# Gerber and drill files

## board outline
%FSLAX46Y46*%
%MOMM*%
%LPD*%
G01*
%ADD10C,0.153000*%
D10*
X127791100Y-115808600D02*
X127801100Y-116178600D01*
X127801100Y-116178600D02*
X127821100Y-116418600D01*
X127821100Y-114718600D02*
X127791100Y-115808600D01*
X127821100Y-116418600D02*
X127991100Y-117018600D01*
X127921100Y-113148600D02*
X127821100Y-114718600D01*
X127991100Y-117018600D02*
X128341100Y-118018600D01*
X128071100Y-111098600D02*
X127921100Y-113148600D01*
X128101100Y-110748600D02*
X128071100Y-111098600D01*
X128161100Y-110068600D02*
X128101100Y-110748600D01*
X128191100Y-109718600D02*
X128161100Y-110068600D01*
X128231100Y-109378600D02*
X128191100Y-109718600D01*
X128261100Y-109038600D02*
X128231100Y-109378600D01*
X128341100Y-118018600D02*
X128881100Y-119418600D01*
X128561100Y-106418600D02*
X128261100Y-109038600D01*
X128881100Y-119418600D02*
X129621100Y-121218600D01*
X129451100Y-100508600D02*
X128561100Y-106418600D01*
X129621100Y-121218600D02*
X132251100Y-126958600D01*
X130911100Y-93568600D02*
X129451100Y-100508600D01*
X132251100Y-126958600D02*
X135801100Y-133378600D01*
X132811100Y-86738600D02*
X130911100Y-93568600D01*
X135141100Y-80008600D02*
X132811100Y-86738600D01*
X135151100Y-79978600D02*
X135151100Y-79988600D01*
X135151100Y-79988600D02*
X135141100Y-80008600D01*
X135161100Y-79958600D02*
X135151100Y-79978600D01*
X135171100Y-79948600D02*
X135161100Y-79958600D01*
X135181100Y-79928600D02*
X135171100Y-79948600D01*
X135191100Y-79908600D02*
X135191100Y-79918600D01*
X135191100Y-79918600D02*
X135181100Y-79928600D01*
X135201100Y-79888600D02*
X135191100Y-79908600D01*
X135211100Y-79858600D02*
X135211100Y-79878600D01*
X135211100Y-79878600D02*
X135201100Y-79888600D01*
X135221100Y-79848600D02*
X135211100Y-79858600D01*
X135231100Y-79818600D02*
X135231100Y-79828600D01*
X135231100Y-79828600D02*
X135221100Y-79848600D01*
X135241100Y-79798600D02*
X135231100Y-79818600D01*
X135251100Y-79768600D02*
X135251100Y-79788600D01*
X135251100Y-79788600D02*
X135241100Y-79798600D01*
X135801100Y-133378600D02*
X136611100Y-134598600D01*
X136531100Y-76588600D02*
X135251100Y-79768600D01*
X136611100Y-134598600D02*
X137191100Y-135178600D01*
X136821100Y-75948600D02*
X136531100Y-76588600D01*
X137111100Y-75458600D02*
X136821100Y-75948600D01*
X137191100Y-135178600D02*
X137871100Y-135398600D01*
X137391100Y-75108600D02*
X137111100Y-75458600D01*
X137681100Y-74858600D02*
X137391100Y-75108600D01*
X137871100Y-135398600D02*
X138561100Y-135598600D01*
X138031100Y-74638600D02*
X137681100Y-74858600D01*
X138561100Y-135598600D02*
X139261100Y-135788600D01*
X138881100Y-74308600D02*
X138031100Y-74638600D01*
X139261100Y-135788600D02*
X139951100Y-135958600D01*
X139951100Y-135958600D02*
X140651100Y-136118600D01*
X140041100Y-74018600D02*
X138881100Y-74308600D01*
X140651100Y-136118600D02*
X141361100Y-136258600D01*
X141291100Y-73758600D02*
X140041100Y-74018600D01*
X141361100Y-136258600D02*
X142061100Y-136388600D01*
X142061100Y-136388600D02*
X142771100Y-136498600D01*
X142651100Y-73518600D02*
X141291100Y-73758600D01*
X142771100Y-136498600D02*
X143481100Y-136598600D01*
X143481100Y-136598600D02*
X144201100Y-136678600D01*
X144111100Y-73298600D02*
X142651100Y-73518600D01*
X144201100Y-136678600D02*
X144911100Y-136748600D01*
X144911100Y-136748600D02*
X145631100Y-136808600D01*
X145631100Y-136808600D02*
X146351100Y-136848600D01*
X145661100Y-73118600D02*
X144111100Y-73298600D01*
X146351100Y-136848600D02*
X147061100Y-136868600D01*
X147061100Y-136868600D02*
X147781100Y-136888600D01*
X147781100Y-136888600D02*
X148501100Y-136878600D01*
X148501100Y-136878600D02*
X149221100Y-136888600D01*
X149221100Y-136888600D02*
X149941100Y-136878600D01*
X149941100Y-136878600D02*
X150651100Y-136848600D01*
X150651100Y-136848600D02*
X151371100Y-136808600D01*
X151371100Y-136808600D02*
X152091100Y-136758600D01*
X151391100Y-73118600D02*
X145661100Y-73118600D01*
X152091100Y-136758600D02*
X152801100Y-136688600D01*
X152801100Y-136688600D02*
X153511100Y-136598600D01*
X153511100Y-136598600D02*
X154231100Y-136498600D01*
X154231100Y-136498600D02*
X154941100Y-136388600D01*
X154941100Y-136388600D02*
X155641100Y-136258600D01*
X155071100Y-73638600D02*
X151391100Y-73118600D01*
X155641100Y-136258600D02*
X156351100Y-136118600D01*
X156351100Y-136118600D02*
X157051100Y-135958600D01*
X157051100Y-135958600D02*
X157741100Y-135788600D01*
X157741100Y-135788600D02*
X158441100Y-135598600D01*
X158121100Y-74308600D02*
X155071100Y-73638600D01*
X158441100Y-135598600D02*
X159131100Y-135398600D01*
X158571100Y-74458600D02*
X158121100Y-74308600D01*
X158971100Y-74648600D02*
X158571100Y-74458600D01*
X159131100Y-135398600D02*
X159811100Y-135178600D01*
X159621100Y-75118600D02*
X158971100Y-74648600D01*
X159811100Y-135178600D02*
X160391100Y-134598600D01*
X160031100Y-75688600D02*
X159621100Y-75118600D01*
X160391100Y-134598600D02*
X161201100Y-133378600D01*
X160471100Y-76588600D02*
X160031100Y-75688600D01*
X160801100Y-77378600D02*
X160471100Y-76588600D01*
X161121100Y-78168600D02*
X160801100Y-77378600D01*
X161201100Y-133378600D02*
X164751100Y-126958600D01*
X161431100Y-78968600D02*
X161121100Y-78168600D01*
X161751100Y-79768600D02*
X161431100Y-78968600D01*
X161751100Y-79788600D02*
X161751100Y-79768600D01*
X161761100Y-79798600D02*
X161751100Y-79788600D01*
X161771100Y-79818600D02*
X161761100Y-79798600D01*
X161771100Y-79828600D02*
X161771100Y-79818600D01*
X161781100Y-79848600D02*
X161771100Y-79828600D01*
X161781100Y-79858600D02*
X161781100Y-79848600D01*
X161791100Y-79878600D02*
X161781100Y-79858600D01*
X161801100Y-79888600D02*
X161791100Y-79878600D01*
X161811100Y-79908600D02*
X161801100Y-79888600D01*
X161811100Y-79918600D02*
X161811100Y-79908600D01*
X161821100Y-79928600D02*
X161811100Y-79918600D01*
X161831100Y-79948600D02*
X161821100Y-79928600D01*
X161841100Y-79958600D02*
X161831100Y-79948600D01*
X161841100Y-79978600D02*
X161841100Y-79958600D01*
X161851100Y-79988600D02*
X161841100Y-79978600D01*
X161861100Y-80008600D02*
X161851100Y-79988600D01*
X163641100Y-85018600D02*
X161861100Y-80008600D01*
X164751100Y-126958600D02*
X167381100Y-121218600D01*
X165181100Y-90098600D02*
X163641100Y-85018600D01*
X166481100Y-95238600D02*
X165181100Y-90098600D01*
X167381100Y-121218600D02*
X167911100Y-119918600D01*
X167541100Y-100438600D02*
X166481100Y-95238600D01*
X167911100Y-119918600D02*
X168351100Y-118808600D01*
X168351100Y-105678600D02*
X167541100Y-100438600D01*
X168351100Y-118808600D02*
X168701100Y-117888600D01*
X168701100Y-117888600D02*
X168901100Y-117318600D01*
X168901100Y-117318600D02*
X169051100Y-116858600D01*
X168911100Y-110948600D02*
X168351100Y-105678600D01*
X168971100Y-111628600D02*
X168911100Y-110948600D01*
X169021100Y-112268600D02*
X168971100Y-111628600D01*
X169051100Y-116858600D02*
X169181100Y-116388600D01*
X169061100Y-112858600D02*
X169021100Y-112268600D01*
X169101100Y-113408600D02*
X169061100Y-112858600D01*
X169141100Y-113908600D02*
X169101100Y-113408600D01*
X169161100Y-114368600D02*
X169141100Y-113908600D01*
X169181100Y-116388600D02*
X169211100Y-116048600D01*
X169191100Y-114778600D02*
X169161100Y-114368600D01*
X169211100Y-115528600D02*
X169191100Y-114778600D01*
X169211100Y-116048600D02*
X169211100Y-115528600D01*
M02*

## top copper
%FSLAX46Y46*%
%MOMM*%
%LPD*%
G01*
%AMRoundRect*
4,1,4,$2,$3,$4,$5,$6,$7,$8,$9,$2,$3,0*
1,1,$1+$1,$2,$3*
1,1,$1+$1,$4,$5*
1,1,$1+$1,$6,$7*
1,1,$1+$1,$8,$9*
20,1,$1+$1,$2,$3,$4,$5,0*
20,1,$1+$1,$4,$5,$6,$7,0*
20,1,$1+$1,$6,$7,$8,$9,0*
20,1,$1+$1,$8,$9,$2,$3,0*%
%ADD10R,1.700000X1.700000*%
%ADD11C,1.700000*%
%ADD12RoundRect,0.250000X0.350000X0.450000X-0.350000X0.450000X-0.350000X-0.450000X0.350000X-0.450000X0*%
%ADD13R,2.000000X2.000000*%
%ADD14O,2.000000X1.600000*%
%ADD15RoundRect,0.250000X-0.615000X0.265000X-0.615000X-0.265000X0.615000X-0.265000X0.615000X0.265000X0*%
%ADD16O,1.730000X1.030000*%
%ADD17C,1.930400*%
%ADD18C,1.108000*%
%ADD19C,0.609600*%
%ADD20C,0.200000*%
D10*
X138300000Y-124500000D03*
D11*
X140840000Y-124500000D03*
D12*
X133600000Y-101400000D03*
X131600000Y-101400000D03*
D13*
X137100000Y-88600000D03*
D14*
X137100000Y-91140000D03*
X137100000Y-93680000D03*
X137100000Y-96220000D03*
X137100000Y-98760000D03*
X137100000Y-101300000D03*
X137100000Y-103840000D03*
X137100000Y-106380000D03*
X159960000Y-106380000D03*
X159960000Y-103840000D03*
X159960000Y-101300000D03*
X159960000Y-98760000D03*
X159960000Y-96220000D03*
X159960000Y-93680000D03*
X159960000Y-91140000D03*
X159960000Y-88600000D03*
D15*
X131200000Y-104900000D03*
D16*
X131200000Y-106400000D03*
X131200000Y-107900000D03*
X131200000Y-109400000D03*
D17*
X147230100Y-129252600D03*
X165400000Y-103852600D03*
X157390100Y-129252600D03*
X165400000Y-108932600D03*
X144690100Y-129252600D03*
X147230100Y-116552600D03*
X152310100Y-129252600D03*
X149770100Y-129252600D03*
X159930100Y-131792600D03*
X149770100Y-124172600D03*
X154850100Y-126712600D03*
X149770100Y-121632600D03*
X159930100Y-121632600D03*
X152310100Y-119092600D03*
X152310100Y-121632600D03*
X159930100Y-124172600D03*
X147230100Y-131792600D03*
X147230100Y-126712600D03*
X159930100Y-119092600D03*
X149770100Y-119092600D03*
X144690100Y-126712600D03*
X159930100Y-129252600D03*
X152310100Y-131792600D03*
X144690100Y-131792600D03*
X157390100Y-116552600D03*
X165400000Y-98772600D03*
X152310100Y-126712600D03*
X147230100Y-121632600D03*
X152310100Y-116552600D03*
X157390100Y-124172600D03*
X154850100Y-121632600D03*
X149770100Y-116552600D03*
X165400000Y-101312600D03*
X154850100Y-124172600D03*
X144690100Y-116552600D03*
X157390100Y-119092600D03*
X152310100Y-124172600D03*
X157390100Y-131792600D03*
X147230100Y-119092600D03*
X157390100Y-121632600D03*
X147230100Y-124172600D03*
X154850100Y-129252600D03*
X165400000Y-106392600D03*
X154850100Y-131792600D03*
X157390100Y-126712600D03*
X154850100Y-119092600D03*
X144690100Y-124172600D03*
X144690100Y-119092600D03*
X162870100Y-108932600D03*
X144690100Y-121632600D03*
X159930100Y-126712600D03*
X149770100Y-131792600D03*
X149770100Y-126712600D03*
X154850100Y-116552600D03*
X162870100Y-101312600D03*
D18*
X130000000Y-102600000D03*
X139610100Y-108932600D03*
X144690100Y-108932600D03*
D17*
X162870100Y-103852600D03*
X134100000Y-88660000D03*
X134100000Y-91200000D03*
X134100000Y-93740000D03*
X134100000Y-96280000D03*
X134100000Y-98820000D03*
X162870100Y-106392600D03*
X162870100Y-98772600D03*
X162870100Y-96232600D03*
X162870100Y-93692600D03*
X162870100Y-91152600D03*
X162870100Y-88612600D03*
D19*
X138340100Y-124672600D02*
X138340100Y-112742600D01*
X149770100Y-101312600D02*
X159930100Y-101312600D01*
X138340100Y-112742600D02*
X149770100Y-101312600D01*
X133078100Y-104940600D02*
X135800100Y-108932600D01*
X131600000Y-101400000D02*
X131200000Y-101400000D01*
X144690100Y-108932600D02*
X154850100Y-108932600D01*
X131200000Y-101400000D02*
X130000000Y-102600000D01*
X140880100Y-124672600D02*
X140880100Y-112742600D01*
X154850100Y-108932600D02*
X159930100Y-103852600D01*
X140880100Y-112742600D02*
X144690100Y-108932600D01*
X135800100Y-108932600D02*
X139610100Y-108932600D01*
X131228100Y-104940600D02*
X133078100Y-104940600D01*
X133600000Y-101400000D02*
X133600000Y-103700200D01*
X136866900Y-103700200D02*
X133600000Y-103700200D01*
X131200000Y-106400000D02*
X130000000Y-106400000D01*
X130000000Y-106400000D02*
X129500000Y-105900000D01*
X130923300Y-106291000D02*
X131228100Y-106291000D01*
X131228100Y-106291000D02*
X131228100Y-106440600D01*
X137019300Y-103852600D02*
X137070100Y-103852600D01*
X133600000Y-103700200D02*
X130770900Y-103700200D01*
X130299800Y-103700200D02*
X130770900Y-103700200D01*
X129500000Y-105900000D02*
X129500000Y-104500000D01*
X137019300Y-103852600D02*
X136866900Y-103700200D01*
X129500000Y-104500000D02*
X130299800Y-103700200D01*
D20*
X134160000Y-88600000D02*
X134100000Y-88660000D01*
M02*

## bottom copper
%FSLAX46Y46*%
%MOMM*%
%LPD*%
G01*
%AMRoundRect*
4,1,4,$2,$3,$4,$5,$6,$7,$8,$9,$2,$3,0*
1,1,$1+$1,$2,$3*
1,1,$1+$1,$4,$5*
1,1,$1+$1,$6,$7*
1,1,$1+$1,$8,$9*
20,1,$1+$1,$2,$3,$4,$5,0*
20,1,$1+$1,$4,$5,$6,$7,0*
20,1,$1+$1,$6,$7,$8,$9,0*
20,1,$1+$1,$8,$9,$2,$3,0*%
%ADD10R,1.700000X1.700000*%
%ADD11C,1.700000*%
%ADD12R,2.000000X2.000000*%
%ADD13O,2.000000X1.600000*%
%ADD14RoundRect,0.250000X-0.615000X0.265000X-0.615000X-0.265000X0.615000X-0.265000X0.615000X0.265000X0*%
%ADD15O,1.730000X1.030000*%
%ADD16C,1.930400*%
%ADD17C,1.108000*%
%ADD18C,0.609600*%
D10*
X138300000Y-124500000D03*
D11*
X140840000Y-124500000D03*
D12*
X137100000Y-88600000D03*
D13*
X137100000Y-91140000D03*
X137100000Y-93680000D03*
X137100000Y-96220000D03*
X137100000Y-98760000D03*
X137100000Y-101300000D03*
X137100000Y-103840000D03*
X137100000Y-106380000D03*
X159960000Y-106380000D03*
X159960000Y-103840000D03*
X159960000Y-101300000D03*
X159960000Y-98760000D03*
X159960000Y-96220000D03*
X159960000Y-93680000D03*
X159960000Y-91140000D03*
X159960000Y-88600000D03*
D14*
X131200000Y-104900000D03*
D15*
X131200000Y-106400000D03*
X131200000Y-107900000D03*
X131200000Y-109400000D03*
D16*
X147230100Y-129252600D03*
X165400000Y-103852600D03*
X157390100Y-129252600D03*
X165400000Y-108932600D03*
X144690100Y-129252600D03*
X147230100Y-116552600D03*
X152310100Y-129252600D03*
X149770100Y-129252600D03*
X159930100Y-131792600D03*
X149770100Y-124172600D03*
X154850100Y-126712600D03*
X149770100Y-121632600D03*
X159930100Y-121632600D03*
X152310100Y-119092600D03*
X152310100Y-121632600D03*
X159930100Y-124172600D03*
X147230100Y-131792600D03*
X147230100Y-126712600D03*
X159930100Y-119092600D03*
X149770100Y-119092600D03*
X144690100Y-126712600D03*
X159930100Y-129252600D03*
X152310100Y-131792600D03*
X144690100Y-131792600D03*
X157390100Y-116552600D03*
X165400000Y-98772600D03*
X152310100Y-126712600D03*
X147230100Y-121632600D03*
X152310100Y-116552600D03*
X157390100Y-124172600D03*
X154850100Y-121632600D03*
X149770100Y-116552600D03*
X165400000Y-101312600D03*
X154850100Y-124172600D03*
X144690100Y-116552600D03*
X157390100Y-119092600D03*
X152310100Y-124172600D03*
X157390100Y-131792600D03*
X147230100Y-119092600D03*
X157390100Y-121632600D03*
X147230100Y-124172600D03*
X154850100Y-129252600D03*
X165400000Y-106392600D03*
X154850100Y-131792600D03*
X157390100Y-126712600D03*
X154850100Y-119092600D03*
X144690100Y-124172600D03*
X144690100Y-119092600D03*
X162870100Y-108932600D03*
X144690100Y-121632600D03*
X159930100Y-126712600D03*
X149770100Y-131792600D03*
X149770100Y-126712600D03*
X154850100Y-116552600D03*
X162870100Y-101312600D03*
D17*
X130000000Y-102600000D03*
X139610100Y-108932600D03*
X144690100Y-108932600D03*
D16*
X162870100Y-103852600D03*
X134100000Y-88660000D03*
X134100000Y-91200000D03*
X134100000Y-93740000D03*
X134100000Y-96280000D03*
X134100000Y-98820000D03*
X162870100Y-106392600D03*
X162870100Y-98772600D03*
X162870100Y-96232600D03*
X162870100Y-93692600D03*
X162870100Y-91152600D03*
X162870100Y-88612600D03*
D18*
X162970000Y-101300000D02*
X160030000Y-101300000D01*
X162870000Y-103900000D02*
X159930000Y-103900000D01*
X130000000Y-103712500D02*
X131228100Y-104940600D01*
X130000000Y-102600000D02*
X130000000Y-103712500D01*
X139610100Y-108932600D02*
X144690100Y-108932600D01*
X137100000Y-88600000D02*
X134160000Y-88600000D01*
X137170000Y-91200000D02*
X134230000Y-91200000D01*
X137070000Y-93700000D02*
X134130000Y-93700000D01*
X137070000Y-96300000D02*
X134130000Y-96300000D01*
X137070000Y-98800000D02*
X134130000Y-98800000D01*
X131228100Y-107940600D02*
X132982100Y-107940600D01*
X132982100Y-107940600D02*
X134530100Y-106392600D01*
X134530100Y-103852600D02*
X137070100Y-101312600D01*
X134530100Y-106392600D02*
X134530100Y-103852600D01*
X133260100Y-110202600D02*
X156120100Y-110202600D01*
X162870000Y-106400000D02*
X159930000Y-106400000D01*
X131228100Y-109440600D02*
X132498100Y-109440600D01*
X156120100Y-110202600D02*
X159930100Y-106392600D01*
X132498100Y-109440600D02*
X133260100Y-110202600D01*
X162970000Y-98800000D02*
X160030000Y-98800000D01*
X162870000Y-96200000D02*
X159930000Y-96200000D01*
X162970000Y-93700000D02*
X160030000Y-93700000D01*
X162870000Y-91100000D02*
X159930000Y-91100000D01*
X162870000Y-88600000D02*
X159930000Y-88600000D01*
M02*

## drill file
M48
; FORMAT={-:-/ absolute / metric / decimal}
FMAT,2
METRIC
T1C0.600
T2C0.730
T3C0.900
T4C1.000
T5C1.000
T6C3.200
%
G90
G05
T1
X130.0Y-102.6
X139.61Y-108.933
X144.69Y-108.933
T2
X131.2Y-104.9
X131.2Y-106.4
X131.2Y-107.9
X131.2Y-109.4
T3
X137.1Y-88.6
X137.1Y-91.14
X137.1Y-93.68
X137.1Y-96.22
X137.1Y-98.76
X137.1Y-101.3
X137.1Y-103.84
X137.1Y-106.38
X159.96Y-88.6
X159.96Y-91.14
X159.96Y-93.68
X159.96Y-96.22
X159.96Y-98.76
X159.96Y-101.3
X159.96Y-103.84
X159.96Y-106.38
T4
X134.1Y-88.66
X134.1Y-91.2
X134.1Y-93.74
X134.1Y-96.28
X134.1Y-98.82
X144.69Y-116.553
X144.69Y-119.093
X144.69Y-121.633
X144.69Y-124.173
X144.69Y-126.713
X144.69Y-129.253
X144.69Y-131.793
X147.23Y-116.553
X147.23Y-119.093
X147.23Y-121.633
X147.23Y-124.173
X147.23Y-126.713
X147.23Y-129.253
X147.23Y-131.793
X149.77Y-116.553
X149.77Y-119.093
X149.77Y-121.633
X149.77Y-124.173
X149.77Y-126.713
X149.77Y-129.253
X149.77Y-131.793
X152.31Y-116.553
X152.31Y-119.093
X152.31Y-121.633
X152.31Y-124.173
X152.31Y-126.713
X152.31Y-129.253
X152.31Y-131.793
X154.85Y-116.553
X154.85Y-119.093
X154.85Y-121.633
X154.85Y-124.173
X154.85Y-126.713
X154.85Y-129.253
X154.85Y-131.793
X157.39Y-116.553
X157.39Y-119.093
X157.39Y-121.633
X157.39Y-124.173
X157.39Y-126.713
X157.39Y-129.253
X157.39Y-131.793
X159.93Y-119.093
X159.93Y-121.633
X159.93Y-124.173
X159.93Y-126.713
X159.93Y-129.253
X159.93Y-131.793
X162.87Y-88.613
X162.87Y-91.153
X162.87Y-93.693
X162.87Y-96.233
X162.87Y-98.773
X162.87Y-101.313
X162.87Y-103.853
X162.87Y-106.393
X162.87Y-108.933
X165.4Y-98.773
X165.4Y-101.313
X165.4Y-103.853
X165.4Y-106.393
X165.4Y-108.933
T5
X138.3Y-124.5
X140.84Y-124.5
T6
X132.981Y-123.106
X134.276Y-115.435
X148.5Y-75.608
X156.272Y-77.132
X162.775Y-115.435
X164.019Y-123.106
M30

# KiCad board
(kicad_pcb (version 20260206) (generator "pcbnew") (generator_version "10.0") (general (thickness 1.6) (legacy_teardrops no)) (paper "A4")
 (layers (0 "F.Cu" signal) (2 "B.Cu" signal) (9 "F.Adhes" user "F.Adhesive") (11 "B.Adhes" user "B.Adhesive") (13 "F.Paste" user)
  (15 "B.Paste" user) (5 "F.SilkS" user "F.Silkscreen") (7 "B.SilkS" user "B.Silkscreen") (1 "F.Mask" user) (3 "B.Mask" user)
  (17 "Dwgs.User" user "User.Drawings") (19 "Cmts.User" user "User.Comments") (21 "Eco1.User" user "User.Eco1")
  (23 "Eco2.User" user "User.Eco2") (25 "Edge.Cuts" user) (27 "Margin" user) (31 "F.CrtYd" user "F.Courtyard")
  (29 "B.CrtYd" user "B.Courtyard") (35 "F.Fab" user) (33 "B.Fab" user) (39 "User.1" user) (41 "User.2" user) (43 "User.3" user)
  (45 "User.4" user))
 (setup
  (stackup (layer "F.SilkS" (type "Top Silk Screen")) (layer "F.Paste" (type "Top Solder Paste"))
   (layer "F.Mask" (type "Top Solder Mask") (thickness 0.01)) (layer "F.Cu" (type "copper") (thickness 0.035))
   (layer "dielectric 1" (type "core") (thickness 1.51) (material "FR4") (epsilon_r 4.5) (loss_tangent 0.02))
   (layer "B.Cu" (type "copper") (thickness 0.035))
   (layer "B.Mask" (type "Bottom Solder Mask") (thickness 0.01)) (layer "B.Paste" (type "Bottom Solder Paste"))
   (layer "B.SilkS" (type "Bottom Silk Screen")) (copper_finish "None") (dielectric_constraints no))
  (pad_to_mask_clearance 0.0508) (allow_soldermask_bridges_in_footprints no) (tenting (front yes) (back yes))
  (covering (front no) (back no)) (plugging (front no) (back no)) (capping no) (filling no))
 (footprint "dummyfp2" (layer "F.Cu") (at 162.7749 115.435)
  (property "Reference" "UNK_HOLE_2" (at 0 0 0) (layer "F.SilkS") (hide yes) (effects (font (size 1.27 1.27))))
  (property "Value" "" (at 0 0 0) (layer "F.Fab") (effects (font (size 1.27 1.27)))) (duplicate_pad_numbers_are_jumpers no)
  (pad "" np_thru_hole circle (at 0 0) (size 3.2 3.2) (drill 3.2) (layers "*.Cu" "*.Mask")))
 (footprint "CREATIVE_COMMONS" (layer "F.Cu") (at 112.9401 148.3026)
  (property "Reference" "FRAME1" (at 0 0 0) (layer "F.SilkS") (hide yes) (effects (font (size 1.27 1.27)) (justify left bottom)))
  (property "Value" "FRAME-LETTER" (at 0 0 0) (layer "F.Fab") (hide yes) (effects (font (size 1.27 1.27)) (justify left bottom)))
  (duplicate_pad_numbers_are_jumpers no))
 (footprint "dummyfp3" (layer "F.Cu") (at 132.9807 123.1058)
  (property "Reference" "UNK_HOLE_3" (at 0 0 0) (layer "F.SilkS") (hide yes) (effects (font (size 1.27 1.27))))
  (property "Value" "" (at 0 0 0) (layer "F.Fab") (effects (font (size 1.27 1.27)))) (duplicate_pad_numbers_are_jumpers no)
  (pad "" np_thru_hole circle (at 0 0) (size 3.2 3.2) (drill 3.2) (layers "*.Cu" "*.Mask")))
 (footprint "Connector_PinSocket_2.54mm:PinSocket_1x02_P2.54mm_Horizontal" (layer "F.Cu") (at 138.3 124.5 90)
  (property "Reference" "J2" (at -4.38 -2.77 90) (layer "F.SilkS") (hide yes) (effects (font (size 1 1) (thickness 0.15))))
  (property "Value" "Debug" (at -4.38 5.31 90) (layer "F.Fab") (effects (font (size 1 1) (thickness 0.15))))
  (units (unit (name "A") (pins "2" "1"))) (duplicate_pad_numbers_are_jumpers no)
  (pad "1" thru_hole rect (at 0 0 90) (size 1.7 1.7) (drill 1) (layers "*.Cu" "*.Mask") (remove_unused_layers no) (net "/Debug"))
  (pad "2" thru_hole circle (at 0 2.54 90) (size 1.7 1.7) (drill 1) (layers "*.Cu" "*.Mask") (remove_unused_layers no) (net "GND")))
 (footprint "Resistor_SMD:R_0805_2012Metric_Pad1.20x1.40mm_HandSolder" (layer "F.Cu") (at 132.6 101.4 180)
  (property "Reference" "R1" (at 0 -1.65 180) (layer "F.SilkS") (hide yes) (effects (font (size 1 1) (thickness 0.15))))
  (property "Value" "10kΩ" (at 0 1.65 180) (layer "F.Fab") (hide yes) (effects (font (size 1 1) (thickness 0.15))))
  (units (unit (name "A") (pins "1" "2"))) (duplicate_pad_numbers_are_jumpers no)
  (pad "1" smd roundrect (at -1 0 180) (size 1.2 1.4) (layers "F.Cu" "F.Mask" "F.Paste") (roundrect_rratio 0.208333) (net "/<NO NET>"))
  (pad "2" smd roundrect (at 1 0 180) (size 1.2 1.4) (layers "F.Cu" "F.Mask" "F.Paste") (roundrect_rratio 0.208333) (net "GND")))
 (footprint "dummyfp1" (layer "F.Cu") (at 156.2725 77.1318)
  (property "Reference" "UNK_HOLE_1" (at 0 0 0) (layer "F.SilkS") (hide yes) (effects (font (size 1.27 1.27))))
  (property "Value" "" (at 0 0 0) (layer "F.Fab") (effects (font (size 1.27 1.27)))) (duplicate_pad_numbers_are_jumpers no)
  (pad "" np_thru_hole circle (at 0 0) (size 3.2 3.2) (drill 3.2) (layers "*.Cu" "*.Mask")))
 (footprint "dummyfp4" (layer "F.Cu") (at 164.0195 123.1058)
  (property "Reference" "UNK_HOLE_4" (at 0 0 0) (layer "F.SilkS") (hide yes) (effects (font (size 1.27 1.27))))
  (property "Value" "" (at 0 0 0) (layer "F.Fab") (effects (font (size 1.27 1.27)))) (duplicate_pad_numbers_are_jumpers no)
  (pad "" np_thru_hole circle (at 0 0) (size 3.2 3.2) (drill 3.2) (layers "*.Cu" "*.Mask")))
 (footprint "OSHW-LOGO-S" (layer "F.Cu") (at 142.2 77.2)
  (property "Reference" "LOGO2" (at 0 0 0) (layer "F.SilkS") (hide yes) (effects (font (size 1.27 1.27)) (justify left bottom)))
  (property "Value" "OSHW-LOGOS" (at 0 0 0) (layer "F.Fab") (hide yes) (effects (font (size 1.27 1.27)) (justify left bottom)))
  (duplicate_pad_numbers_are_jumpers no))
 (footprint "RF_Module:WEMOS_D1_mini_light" (layer "F.Cu") (at 137.1 88.6)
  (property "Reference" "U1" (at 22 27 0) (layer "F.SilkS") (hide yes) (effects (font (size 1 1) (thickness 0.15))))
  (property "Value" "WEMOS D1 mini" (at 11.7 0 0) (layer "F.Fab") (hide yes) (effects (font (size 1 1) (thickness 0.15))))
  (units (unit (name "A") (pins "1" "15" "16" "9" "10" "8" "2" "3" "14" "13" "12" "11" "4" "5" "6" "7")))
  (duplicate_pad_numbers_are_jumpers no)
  (pad "1" thru_hole rect (at 0 0) (size 2 2) (drill 0.9) (layers "*.Cu" "*.Mask") (remove_unused_layers no)
   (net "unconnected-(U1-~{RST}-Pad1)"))
  (pad "2" thru_hole oval (at 0 2.54) (size 2 1.6) (drill 0.9) (layers "*.Cu" "*.Mask") (remove_unused_layers no)
   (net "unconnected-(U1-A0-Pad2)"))
  (pad "3" thru_hole oval (at 0 5.08) (size 2 1.6) (drill 0.9) (layers "*.Cu" "*.Mask") (remove_unused_layers no)
   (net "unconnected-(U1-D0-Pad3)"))
  (pad "4" thru_hole oval (at 0 7.62) (size 2 1.6) (drill 0.9) (layers "*.Cu" "*.Mask") (remove_unused_layers no)
   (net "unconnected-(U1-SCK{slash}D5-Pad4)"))
  (pad "5" thru_hole oval (at 0 10.16) (size 2 1.6) (drill 0.9) (layers "*.Cu" "*.Mask") (remove_unused_layers no)
   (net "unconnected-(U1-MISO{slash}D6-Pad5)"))
  (pad "6" thru_hole oval (at 0 12.7) (size 2 1.6) (drill 0.9) (layers "*.Cu" "*.Mask") (remove_unused_layers no) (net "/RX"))
  (pad "7" thru_hole oval (at 0 15.24) (size 2 1.6) (drill 0.9) (layers "*.Cu" "*.Mask") (remove_unused_layers no) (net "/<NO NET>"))
  (pad "8" thru_hole oval (at 0 17.78) (size 2 1.6) (drill 0.9) (layers "*.Cu" "*.Mask") (remove_unused_layers no)
   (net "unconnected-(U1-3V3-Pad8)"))
  (pad "9" thru_hole oval (at 22.86 17.78) (size 2 1.6) (drill 0.9) (layers "*.Cu" "*.Mask") (remove_unused_layers no) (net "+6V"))
  (pad "10" thru_hole oval (at 22.86 15.24) (size 2 1.6) (drill 0.9) (layers "*.Cu" "*.Mask") (remove_unused_layers no) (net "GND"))
  (pad "11" thru_hole oval (at 22.86 12.7) (size 2 1.6) (drill 0.9) (layers "*.Cu" "*.Mask") (remove_unused_layers no) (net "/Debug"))
  (pad "12" thru_hole oval (at 22.86 10.16) (size 2 1.6) (drill 0.9) (layers "*.Cu" "*.Mask") (remove_unused_layers no)
   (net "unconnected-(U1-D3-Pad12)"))
  (pad "13" thru_hole oval (at 22.86 7.62) (size 2 1.6) (drill 0.9) (layers "*.Cu" "*.Mask") (remove_unused_layers no)
   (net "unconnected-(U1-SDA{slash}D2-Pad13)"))
  (pad "14" thru_hole oval (at 22.86 5.08) (size 2 1.6) (drill 0.9) (layers "*.Cu" "*.Mask") (remove_unused_layers no)
   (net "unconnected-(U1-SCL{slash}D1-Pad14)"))
  (pad "15" thru_hole oval (at 22.86 2.54) (size 2 1.6) (drill 0.9) (layers "*.Cu" "*.Mask") (remove_unused_layers no)
   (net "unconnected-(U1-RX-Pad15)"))
  (pad "16" thru_hole oval (at 22.86 0) (size 2 1.6) (drill 0.9) (layers "*.Cu" "*.Mask") (remove_unused_layers no)
   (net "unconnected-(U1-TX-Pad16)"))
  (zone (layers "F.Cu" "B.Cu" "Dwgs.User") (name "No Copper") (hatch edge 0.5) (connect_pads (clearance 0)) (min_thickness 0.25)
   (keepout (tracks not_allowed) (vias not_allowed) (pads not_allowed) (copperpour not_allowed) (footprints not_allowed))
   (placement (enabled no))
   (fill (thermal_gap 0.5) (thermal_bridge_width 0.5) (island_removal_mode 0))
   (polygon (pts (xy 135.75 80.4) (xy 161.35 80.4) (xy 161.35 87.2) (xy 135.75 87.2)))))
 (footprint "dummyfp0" (layer "F.Cu") (at 148.5001 75.6078)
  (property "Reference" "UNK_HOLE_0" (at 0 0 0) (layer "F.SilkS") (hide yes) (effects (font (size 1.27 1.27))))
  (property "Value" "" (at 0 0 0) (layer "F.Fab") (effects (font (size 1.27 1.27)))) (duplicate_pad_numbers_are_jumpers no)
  (pad "" np_thru_hole circle (at 0 0) (size 3.2 3.2) (drill 3.2) (layers "*.Cu" "*.Mask")))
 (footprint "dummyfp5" (layer "F.Cu") (at 134.2761 115.435)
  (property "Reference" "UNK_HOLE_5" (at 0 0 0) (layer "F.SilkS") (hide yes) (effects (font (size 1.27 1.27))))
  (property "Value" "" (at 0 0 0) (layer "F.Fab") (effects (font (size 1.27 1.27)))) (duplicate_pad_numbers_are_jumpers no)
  (pad "" np_thru_hole circle (at 0 0) (size 3.2 3.2) (drill 3.2) (layers "*.Cu" "*.Mask")))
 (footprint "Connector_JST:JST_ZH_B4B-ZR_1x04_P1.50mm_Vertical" (layer "B.Cu") (at 131.2 104.9 -90)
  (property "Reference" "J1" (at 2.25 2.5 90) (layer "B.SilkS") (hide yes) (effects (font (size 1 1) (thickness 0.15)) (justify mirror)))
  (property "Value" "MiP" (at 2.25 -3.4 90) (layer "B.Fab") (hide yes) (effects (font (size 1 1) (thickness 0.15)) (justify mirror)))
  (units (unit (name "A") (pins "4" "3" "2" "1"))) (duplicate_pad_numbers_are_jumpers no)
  (pad "1" thru_hole roundrect (at 0 0 270) (size 1.03 1.73) (drill 0.73) (layers "*.Cu" "*.Mask") (remove_unused_layers no)
   (roundrect_rratio 0.242718) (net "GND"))
  (pad "2" thru_hole oval (at 1.5 0 270) (size 1.03 1.73) (drill 0.73) (layers "*.Cu" "*.Mask") (remove_unused_layers no) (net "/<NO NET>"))
  (pad "3" thru_hole oval (at 3 0 270) (size 1.03 1.73) (drill 0.73) (layers "*.Cu" "*.Mask") (remove_unused_layers no) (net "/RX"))
  (pad "4" thru_hole oval (at 4.5 0 270) (size 1.03 1.73) (drill 0.73) (layers "*.Cu" "*.Mask") (remove_unused_layers no) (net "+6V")))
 (gr_line (start 127.7911 115.8086) (end 127.8011 116.1786) (stroke (width 0.153) (type solid)) (layer "Edge.Cuts"))
 (gr_line (start 127.8011 116.1786) (end 127.8211 116.4186) (stroke (width 0.153) (type solid)) (layer "Edge.Cuts"))
 (gr_line (start 127.8211 114.7186) (end 127.7911 115.8086) (stroke (width 0.153) (type solid)) (layer "Edge.Cuts"))
 (gr_line (start 127.8211 116.4186) (end 127.9911 117.0186) (stroke (width 0.153) (type solid)) (layer "Edge.Cuts"))
 (gr_line (start 127.9211 113.1486) (end 127.8211 114.7186) (stroke (width 0.153) (type solid)) (layer "Edge.Cuts"))
 (gr_line (start 127.9911 117.0186) (end 128.3411 118.0186) (stroke (width 0.153) (type solid)) (layer "Edge.Cuts"))
 (gr_line (start 128.0711 111.0986) (end 127.9211 113.1486) (stroke (width 0.153) (type solid)) (layer "Edge.Cuts"))
 (gr_line (start 128.1011 110.7486) (end 128.0711 111.0986) (stroke (width 0.153) (type solid)) (layer "Edge.Cuts"))
 (gr_line (start 128.1611 110.0686) (end 128.1011 110.7486) (stroke (width 0.153) (type solid)) (layer "Edge.Cuts"))
 (gr_line (start 128.1911 109.7186) (end 128.1611 110.0686) (stroke (width 0.153) (type solid)) (layer "Edge.Cuts"))
 (gr_line (start 128.2311 109.3786) (end 128.1911 109.7186) (stroke (width 0.153) (type solid)) (layer "Edge.Cuts"))
 (gr_line (start 128.2611 109.0386) (end 128.2311 109.3786) (stroke (width 0.153) (type solid)) (layer "Edge.Cuts"))
 (gr_line (start 128.3411 118.0186) (end 128.8811 119.4186) (stroke (width 0.153) (type solid)) (layer "Edge.Cuts"))
 (gr_line (start 128.5611 106.4186) (end 128.2611 109.0386) (stroke (width 0.153) (type solid)) (layer "Edge.Cuts"))
 (gr_line (start 128.8811 119.4186) (end 129.6211 121.2186) (stroke (width 0.153) (type solid)) (layer "Edge.Cuts"))
 (gr_line (start 129.4511 100.5086) (end 128.5611 106.4186) (stroke (width 0.153) (type solid)) (layer "Edge.Cuts"))
 (gr_line (start 129.6211 121.2186) (end 132.2511 126.9586) (stroke (width 0.153) (type solid)) (layer "Edge.Cuts"))
 (gr_line (start 130.9111 93.5686) (end 129.4511 100.5086) (stroke (width 0.153) (type solid)) (layer "Edge.Cuts"))
 (gr_line (start 132.2511 126.9586) (end 135.8011 133.3786) (stroke (width 0.153) (type solid)) (layer "Edge.Cuts"))
 (gr_line (start 132.8111 86.7386) (end 130.9111 93.5686) (stroke (width 0.153) (type solid)) (layer "Edge.Cuts"))
 (gr_line (start 135.1411 80.0086) (end 132.8111 86.7386) (stroke (width 0.153) (type solid)) (layer "Edge.Cuts"))
 (gr_line (start 135.1511 79.9786) (end 135.1511 79.9886) (stroke (width 0.153) (type solid)) (layer "Edge.Cuts"))
 (gr_line (start 135.1511 79.9886) (end 135.1411 80.0086) (stroke (width 0.153) (type solid)) (layer "Edge.Cuts"))
 (gr_line (start 135.1611 79.9586) (end 135.1511 79.9786) (stroke (width 0.153) (type solid)) (layer "Edge.Cuts"))
 (gr_line (start 135.1711 79.9486) (end 135.1611 79.9586) (stroke (width 0.153) (type solid)) (layer "Edge.Cuts"))
 (gr_line (start 135.1811 79.9286) (end 135.1711 79.9486) (stroke (width 0.153) (type solid)) (layer "Edge.Cuts"))
 (gr_line (start 135.1911 79.9086) (end 135.1911 79.9186) (stroke (width 0.153) (type solid)) (layer "Edge.Cuts"))
 (gr_line (start 135.1911 79.9186) (end 135.1811 79.9286) (stroke (width 0.153) (type solid)) (layer "Edge.Cuts"))
 (gr_line (start 135.2011 79.8886) (end 135.1911 79.9086) (stroke (width 0.153) (type solid)) (layer "Edge.Cuts"))
 (gr_line (start 135.2111 79.8586) (end 135.2111 79.8786) (stroke (width 0.153) (type solid)) (layer "Edge.Cuts"))
 (gr_line (start 135.2111 79.8786) (end 135.2011 79.8886) (stroke (width 0.153) (type solid)) (layer "Edge.Cuts"))
 (gr_line (start 135.2211 79.8486) (end 135.2111 79.8586) (stroke (width 0.153) (type solid)) (layer "Edge.Cuts"))
 (gr_line (start 135.2311 79.8186) (end 135.2311 79.8286) (stroke (width 0.153) (type solid)) (layer "Edge.Cuts"))
 (gr_line (start 135.2311 79.8286) (end 135.2211 79.8486) (stroke (width 0.153) (type solid)) (layer "Edge.Cuts"))
 (gr_line (start 135.2411 79.7986) (end 135.2311 79.8186) (stroke (width 0.153) (type solid)) (layer "Edge.Cuts"))
 (gr_line (start 135.2511 79.7686) (end 135.2511 79.7886) (stroke (width 0.153) (type solid)) (layer "Edge.Cuts"))
 (gr_line (start 135.2511 79.7886) (end 135.2411 79.7986) (stroke (width 0.153) (type solid)) (layer "Edge.Cuts"))
 (gr_line (start 135.8011 133.3786) (end 136.6111 134.5986) (stroke (width 0.153) (type solid)) (layer "Edge.Cuts"))
 (gr_line (start 136.5311 76.5886) (end 135.2511 79.7686) (stroke (width 0.153) (type solid)) (layer "Edge.Cuts"))
 (gr_line (start 136.6111 134.5986) (end 137.1911 135.1786) (stroke (width 0.153) (type solid)) (layer "Edge.Cuts"))
 (gr_line (start 136.8211 75.9486) (end 136.5311 76.5886) (stroke (width 0.153) (type solid)) (layer "Edge.Cuts"))
 (gr_line (start 137.1111 75.4586) (end 136.8211 75.9486) (stroke (width 0.153) (type solid)) (layer "Edge.Cuts"))
 (gr_line (start 137.1911 135.1786) (end 137.8711 135.3986) (stroke (width 0.153) (type solid)) (layer "Edge.Cuts"))
 (gr_line (start 137.3911 75.1086) (end 137.1111 75.4586) (stroke (width 0.153) (type solid)) (layer "Edge.Cuts"))
 (gr_line (start 137.6811 74.8586) (end 137.3911 75.1086) (stroke (width 0.153) (type solid)) (layer "Edge.Cuts"))
 (gr_line (start 137.8711 135.3986) (end 138.5611 135.5986) (stroke (width 0.153) (type solid)) (layer "Edge.Cuts"))
 (gr_line (start 138.0311 74.6386) (end 137.6811 74.8586) (stroke (width 0.153) (type solid)) (layer "Edge.Cuts"))
 (gr_line (start 138.5611 135.5986) (end 139.2611 135.7886) (stroke (width 0.153) (type solid)) (layer "Edge.Cuts"))
 (gr_line (start 138.8811 74.3086) (end 138.0311 74.6386) (stroke (width 0.153) (type solid)) (layer "Edge.Cuts"))
 (gr_line (start 139.2611 135.7886) (end 139.9511 135.9586) (stroke (width 0.153) (type solid)) (layer "Edge.Cuts"))
 (gr_line (start 139.9511 135.9586) (end 140.6511 136.1186) (stroke (width 0.153) (type solid)) (layer "Edge.Cuts"))
 (gr_line (start 140.0411 74.0186) (end 138.8811 74.3086) (stroke (width 0.153) (type solid)) (layer "Edge.Cuts"))
 (gr_line (start 140.6511 136.1186) (end 141.3611 136.2586) (stroke (width 0.153) (type solid)) (layer "Edge.Cuts"))
 (gr_line (start 141.2911 73.7586) (end 140.0411 74.0186) (stroke (width 0.153) (type solid)) (layer "Edge.Cuts"))
 (gr_line (start 141.3611 136.2586) (end 142.0611 136.3886) (stroke (width 0.153) (type solid)) (layer "Edge.Cuts"))
 (gr_line (start 142.0611 136.3886) (end 142.7711 136.4986) (stroke (width 0.153) (type solid)) (layer "Edge.Cuts"))
 (gr_line (start 142.6511 73.5186) (end 141.2911 73.7586) (stroke (width 0.153) (type solid)) (layer "Edge.Cuts"))
 (gr_line (start 142.7711 136.4986) (end 143.4811 136.5986) (stroke (width 0.153) (type solid)) (layer "Edge.Cuts"))
 (gr_line (start 143.4811 136.5986) (end 144.2011 136.6786) (stroke (width 0.153) (type solid)) (layer "Edge.Cuts"))
 (gr_line (start 144.1111 73.2986) (end 142.6511 73.5186) (stroke (width 0.153) (type solid)) (layer "Edge.Cuts"))
 (gr_line (start 144.2011 136.6786) (end 144.9111 136.7486) (stroke (width 0.153) (type solid)) (layer "Edge.Cuts"))
 (gr_line (start 144.9111 136.7486) (end 145.6311 136.8086) (stroke (width 0.153) (type solid)) (layer "Edge.Cuts"))
 (gr_line (start 145.6311 136.8086) (end 146.3511 136.8486) (stroke (width 0.153) (type solid)) (layer "Edge.Cuts"))
 (gr_line (start 145.6611 73.1186) (end 144.1111 73.2986) (stroke (width 0.153) (type solid)) (layer "Edge.Cuts"))
 (gr_line (start 146.3511 136.8486) (end 147.0611 136.8686) (stroke (width 0.153) (type solid)) (layer "Edge.Cuts"))
 (gr_line (start 147.0611 136.8686) (end 147.7811 136.8886) (stroke (width 0.153) (type solid)) (layer "Edge.Cuts"))
 (gr_line (start 147.7811 136.8886) (end 148.5011 136.8786) (stroke (width 0.153) (type solid)) (layer "Edge.Cuts"))
 (gr_line (start 148.5011 136.8786) (end 149.2211 136.8886) (stroke (width 0.153) (type solid)) (layer "Edge.Cuts"))
 (gr_line (start 149.2211 136.8886) (end 149.9411 136.8786) (stroke (width 0.153) (type solid)) (layer "Edge.Cuts"))
 (gr_line (start 149.9411 136.8786) (end 150.6511 136.8486) (stroke (width 0.153) (type solid)) (layer "Edge.Cuts"))
 (gr_line (start 150.6511 136.8486) (end 151.3711 136.8086) (stroke (width 0.153) (type solid)) (layer "Edge.Cuts"))
 (gr_line (start 151.3711 136.8086) (end 152.0911 136.7586) (stroke (width 0.153) (type solid)) (layer "Edge.Cuts"))
 (gr_line (start 151.3911 73.1186) (end 145.6611 73.1186) (stroke (width 0.153) (type solid)) (layer "Edge.Cuts"))
 (gr_line (start 152.0911 136.7586) (end 152.8011 136.6886) (stroke (width 0.153) (type solid)) (layer "Edge.Cuts"))
 (gr_line (start 152.8011 136.6886) (end 153.5111 136.5986) (stroke (width 0.153) (type solid)) (layer "Edge.Cuts"))
 (gr_line (start 153.5111 136.5986) (end 154.2311 136.4986) (stroke (width 0.153) (type solid)) (layer "Edge.Cuts"))
 (gr_line (start 154.2311 136.4986) (end 154.9411 136.3886) (stroke (width 0.153) (type solid)) (layer "Edge.Cuts"))
 (gr_line (start 154.9411 136.3886) (end 155.6411 136.2586) (stroke (width 0.153) (type solid)) (layer "Edge.Cuts"))
 (gr_line (start 155.0711 73.6386) (end 151.3911 73.1186) (stroke (width 0.153) (type solid)) (layer "Edge.Cuts"))
 (gr_line (start 155.6411 136.2586) (end 156.3511 136.1186) (stroke (width 0.153) (type solid)) (layer "Edge.Cuts"))
 (gr_line (start 156.3511 136.1186) (end 157.0511 135.9586) (stroke (width 0.153) (type solid)) (layer "Edge.Cuts"))
 (gr_line (start 157.0511 135.9586) (end 157.7411 135.7886) (stroke (width 0.153) (type solid)) (layer "Edge.Cuts"))
 (gr_line (start 157.7411 135.7886) (end 158.4411 135.5986) (stroke (width 0.153) (type solid)) (layer "Edge.Cuts"))
 (gr_line (start 158.1211 74.3086) (end 155.0711 73.6386) (stroke (width 0.153) (type solid)) (layer "Edge.Cuts"))
 (gr_line (start 158.4411 135.5986) (end 159.1311 135.3986) (stroke (width 0.153) (type solid)) (layer "Edge.Cuts"))
 (gr_line (start 158.5711 74.4586) (end 158.1211 74.3086) (stroke (width 0.153) (type solid)) (layer "Edge.Cuts"))
 (gr_line (start 158.9711 74.6486) (end 158.5711 74.4586) (stroke (width 0.153) (type solid)) (layer "Edge.Cuts"))
 (gr_line (start 159.1311 135.3986) (end 159.8111 135.1786) (stroke (width 0.153) (type solid)) (layer "Edge.Cuts"))
 (gr_line (start 159.6211 75.1186) (end 158.9711 74.6486) (stroke (width 0.153) (type solid)) (layer "Edge.Cuts"))
 (gr_line (start 159.8111 135.1786) (end 160.3911 134.5986) (stroke (width 0.153) (type solid)) (layer "Edge.Cuts"))
 (gr_line (start 160.0311 75.6886) (end 159.6211 75.1186) (stroke (width 0.153) (type solid)) (layer "Edge.Cuts"))
 (gr_line (start 160.3911 134.5986) (end 161.2011 133.3786) (stroke (width 0.153) (type solid)) (layer "Edge.Cuts"))
 (gr_line (start 160.4711 76.5886) (end 160.0311 75.6886) (stroke (width 0.153) (type solid)) (layer "Edge.Cuts"))
 (gr_line (start 160.8011 77.3786) (end 160.4711 76.5886) (stroke (width 0.153) (type solid)) (layer "Edge.Cuts"))
 (gr_line (start 161.1211 78.1686) (end 160.8011 77.3786) (stroke (width 0.153) (type solid)) (layer "Edge.Cuts"))
 (gr_line (start 161.2011 133.3786) (end 164.7511 126.9586) (stroke (width 0.153) (type solid)) (layer "Edge.Cuts"))
 (gr_line (start 161.4311 78.9686) (end 161.1211 78.1686) (stroke (width 0.153) (type solid)) (layer "Edge.Cuts"))
 (gr_line (start 161.7511 79.7686) (end 161.4311 78.9686) (stroke (width 0.153) (type solid)) (layer "Edge.Cuts"))
 (gr_line (start 161.7511 79.7886) (end 161.7511 79.7686) (stroke (width 0.153) (type solid)) (layer "Edge.Cuts"))
 (gr_line (start 161.7611 79.7986) (end 161.7511 79.7886) (stroke (width 0.153) (type solid)) (layer "Edge.Cuts"))
 (gr_line (start 161.7711 79.8186) (end 161.7611 79.7986) (stroke (width 0.153) (type solid)) (layer "Edge.Cuts"))
 (gr_line (start 161.7711 79.8286) (end 161.7711 79.8186) (stroke (width 0.153) (type solid)) (layer "Edge.Cuts"))
 (gr_line (start 161.7811 79.8486) (end 161.7711 79.8286) (stroke (width 0.153) (type solid)) (layer "Edge.Cuts"))
 (gr_line (start 161.7811 79.8586) (end 161.7811 79.8486) (stroke (width 0.153) (type solid)) (layer "Edge.Cuts"))
 (gr_line (start 161.7911 79.8786) (end 161.7811 79.8586) (stroke (width 0.153) (type solid)) (layer "Edge.Cuts"))
 (gr_line (start 161.8011 79.8886) (end 161.7911 79.8786) (stroke (width 0.153) (type solid)) (layer "Edge.Cuts"))
 (gr_line (start 161.8111 79.9086) (end 161.8011 79.8886) (stroke (width 0.153) (type solid)) (layer "Edge.Cuts"))
 (gr_line (start 161.8111 79.9186) (end 161.8111 79.9086) (stroke (width 0.153) (type solid)) (layer "Edge.Cuts"))
 (gr_line (start 161.8211 79.9286) (end 161.8111 79.9186) (stroke (width 0.153) (type solid)) (layer "Edge.Cuts"))
 (gr_line (start 161.8311 79.9486) (end 161.8211 79.9286) (stroke (width 0.153) (type solid)) (layer "Edge.Cuts"))
 (gr_line (start 161.8411 79.9586) (end 161.8311 79.9486) (stroke (width 0.153) (type solid)) (layer "Edge.Cuts"))
 (gr_line (start 161.8411 79.9786) (end 161.8411 79.9586) (stroke (width 0.153) (type solid)) (layer "Edge.Cuts"))
 (gr_line (start 161.8511 79.9886) (end 161.8411 79.9786) (stroke (width 0.153) (type solid)) (layer "Edge.Cuts"))
 (gr_line (start 161.8611 80.0086) (end 161.8511 79.9886) (stroke (width 0.153) (type solid)) (layer "Edge.Cuts"))
 (gr_line (start 163.6411 85.0186) (end 161.8611 80.0086) (stroke (width 0.153) (type solid)) (layer "Edge.Cuts"))
 (gr_line (start 164.7511 126.9586) (end 167.3811 121.2186) (stroke (width 0.153) (type solid)) (layer "Edge.Cuts"))
 (gr_line (start 165.1811 90.0986) (end 163.6411 85.0186) (stroke (width 0.153) (type solid)) (layer "Edge.Cuts"))
 (gr_line (start 166.4811 95.2386) (end 165.1811 90.0986) (stroke (width 0.153) (type solid)) (layer "Edge.Cuts"))
 (gr_line (start 167.3811 121.2186) (end 167.9111 119.9186) (stroke (width 0.153) (type solid)) (layer "Edge.Cuts"))
 (gr_line (start 167.5411 100.4386) (end 166.4811 95.2386) (stroke (width 0.153) (type solid)) (layer "Edge.Cuts"))
 (gr_line (start 167.9111 119.9186) (end 168.3511 118.8086) (stroke (width 0.153) (type solid)) (layer "Edge.Cuts"))
 (gr_line (start 168.3511 105.6786) (end 167.5411 100.4386) (stroke (width 0.153) (type solid)) (layer "Edge.Cuts"))
 (gr_line (start 168.3511 118.8086) (end 168.7011 117.8886) (stroke (width 0.153) (type solid)) (layer "Edge.Cuts"))
 (gr_line (start 168.7011 117.8886) (end 168.9011 117.3186) (stroke (width 0.153) (type solid)) (layer "Edge.Cuts"))
 (gr_line (start 168.9011 117.3186) (end 169.0511 116.8586) (stroke (width 0.153) (type solid)) (layer "Edge.Cuts"))
 (gr_line (start 168.9111 110.9486) (end 168.3511 105.6786) (stroke (width 0.153) (type solid)) (layer "Edge.Cuts"))
 (gr_line (start 168.9711 111.6286) (end 168.9111 110.9486) (stroke (width 0.153) (type solid)) (layer "Edge.Cuts"))
 (gr_line (start 169.0211 112.2686) (end 168.9711 111.6286) (stroke (width 0.153) (type solid)) (layer "Edge.Cuts"))
 (gr_line (start 169.0511 116.8586) (end 169.1811 116.3886) (stroke (width 0.153) (type solid)) (layer "Edge.Cuts"))
 (gr_line (start 169.0611 112.8586) (end 169.0211 112.2686) (stroke (width 0.153) (type solid)) (layer "Edge.Cuts"))
 (gr_line (start 169.1011 113.4086) (end 169.0611 112.8586) (stroke (width 0.153) (type solid)) (layer "Edge.Cuts"))
 (gr_line (start 169.1411 113.9086) (end 169.1011 113.4086) (stroke (width 0.153) (type solid)) (layer "Edge.Cuts"))
 (gr_line (start 169.1611 114.3686) (end 169.1411 113.9086) (stroke (width 0.153) (type solid)) (layer "Edge.Cuts"))
 (gr_line (start 169.1811 116.3886) (end 169.2111 116.0486) (stroke (width 0.153) (type solid)) (layer "Edge.Cuts"))
 (gr_line (start 169.1911 114.7786) (end 169.1611 114.3686) (stroke (width 0.153) (type solid)) (layer "Edge.Cuts"))
 (gr_line (start 169.2111 115.5286) (end 169.1911 114.7786) (stroke (width 0.153) (type solid)) (layer "Edge.Cuts"))
 (gr_line (start 169.2111 116.0486) (end 169.2111 115.5286) (stroke (width 0.153) (type solid)) (layer "Edge.Cuts"))
 (via (at 147.2301 129.2526) (size 1.9304) (drill 1) (layers "F.Cu" "B.Cu") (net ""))
 (via (at 165.4 103.8526) (size 1.9304) (drill 1) (layers "F.Cu" "B.Cu") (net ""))
 (via (at 157.3901 129.2526) (size 1.9304) (drill 1) (layers "F.Cu" "B.Cu") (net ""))
 (via (at 165.4 108.9326) (size 1.9304) (drill 1) (layers "F.Cu" "B.Cu") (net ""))
 (via (at 144.6901 129.2526) (size 1.9304) (drill 1) (layers "F.Cu" "B.Cu") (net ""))
 (via (at 147.2301 116.5526) (size 1.9304) (drill 1) (layers "F.Cu" "B.Cu") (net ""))
 (via (at 152.3101 129.2526) (size 1.9304) (drill 1) (layers "F.Cu" "B.Cu") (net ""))
 (via (at 149.7701 129.2526) (size 1.9304) (drill 1) (layers "F.Cu" "B.Cu") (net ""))
 (via (at 159.9301 131.7926) (size 1.9304) (drill 1) (layers "F.Cu" "B.Cu") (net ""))
 (via (at 149.7701 124.1726) (size 1.9304) (drill 1) (layers "F.Cu" "B.Cu") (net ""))
 (via (at 154.8501 126.7126) (size 1.9304) (drill 1) (layers "F.Cu" "B.Cu") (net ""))
 (via (at 149.7701 121.6326) (size 1.9304) (drill 1) (layers "F.Cu" "B.Cu") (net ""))
 (via (at 159.9301 121.6326) (size 1.9304) (drill 1) (layers "F.Cu" "B.Cu") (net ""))
 (via (at 152.3101 119.0926) (size 1.9304) (drill 1) (layers "F.Cu" "B.Cu") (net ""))
 (via (at 152.3101 121.6326) (size 1.9304) (drill 1) (layers "F.Cu" "B.Cu") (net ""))
 (via (at 159.9301 124.1726) (size 1.9304) (drill 1) (layers "F.Cu" "B.Cu") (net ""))
 (via (at 147.2301 131.7926) (size 1.9304) (drill 1) (layers "F.Cu" "B.Cu") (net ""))
 (via (at 147.2301 126.7126) (size 1.9304) (drill 1) (layers "F.Cu" "B.Cu") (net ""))
 (via (at 159.9301 119.0926) (size 1.9304) (drill 1) (layers "F.Cu" "B.Cu") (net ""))
 (via (at 149.7701 119.0926) (size 1.9304) (drill 1) (layers "F.Cu" "B.Cu") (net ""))
 (via (at 144.6901 126.7126) (size 1.9304) (drill 1) (layers "F.Cu" "B.Cu") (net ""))
 (via (at 159.9301 129.2526) (size 1.9304) (drill 1) (layers "F.Cu" "B.Cu") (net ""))
 (via (at 152.3101 131.7926) (size 1.9304) (drill 1) (layers "F.Cu" "B.Cu") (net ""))
 (via (at 144.6901 131.7926) (size 1.9304) (drill 1) (layers "F.Cu" "B.Cu") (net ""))
 (via (at 157.3901 116.5526) (size 1.9304) (drill 1) (layers "F.Cu" "B.Cu") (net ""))
 (via (at 165.4 98.7726) (size 1.9304) (drill 1) (layers "F.Cu" "B.Cu") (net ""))
 (via (at 152.3101 126.7126) (size 1.9304) (drill 1) (layers "F.Cu" "B.Cu") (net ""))
 (via (at 147.2301 121.6326) (size 1.9304) (drill 1) (layers "F.Cu" "B.Cu") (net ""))
 (via (at 152.3101 116.5526) (size 1.9304) (drill 1) (layers "F.Cu" "B.Cu") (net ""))
 (via (at 157.3901 124.1726) (size 1.9304) (drill 1) (layers "F.Cu" "B.Cu") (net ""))
 (via (at 154.8501 121.6326) (size 1.9304) (drill 1) (layers "F.Cu" "B.Cu") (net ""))
 (via (at 149.7701 116.5526) (size 1.9304) (drill 1) (layers "F.Cu" "B.Cu") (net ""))
 (via (at 165.4 101.3126) (size 1.9304) (drill 1) (layers "F.Cu" "B.Cu") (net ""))
 (via (at 154.8501 124.1726) (size 1.9304) (drill 1) (layers "F.Cu" "B.Cu") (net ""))
 (via (at 144.6901 116.5526) (size 1.9304) (drill 1) (layers "F.Cu" "B.Cu") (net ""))
 (via (at 157.3901 119.0926) (size 1.9304) (drill 1) (layers "F.Cu" "B.Cu") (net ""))
 (via (at 152.3101 124.1726) (size 1.9304) (drill 1) (layers "F.Cu" "B.Cu") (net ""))
 (via (at 157.3901 131.7926) (size 1.9304) (drill 1) (layers "F.Cu" "B.Cu") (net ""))
 (via (at 147.2301 119.0926) (size 1.9304) (drill 1) (layers "F.Cu" "B.Cu") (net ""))
 (via (at 157.3901 121.6326) (size 1.9304) (drill 1) (layers "F.Cu" "B.Cu") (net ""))
 (via (at 147.2301 124.1726) (size 1.9304) (drill 1) (layers "F.Cu" "B.Cu") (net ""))
 (via (at 154.8501 129.2526) (size 1.9304) (drill 1) (layers "F.Cu" "B.Cu") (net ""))
 (via (at 165.4 106.3926) (size 1.9304) (drill 1) (layers "F.Cu" "B.Cu") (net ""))
 (via (at 154.8501 131.7926) (size 1.9304) (drill 1) (layers "F.Cu" "B.Cu") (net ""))
 (via (at 157.3901 126.7126) (size 1.9304) (drill 1) (layers "F.Cu" "B.Cu") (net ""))
 (via (at 154.8501 119.0926) (size 1.9304) (drill 1) (layers "F.Cu" "B.Cu") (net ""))
 (via (at 144.6901 124.1726) (size 1.9304) (drill 1) (layers "F.Cu" "B.Cu") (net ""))
 (via (at 144.6901 119.0926) (size 1.9304) (drill 1) (layers "F.Cu" "B.Cu") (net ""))
 (via (at 162.8701 108.9326) (size 1.9304) (drill 1) (layers "F.Cu" "B.Cu") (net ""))
 (via (at 144.6901 121.6326) (size 1.9304) (drill 1) (layers "F.Cu" "B.Cu") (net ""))
 (via (at 159.9301 126.7126) (size 1.9304) (drill 1) (layers "F.Cu" "B.Cu") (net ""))
 (via (at 149.7701 131.7926) (size 1.9304) (drill 1) (layers "F.Cu" "B.Cu") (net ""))
 (via (at 149.7701 126.7126) (size 1.9304) (drill 1) (layers "F.Cu" "B.Cu") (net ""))
 (via (at 154.8501 116.5526) (size 1.9304) (drill 1) (layers "F.Cu" "B.Cu") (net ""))
 (segment (start 138.3401 124.6726) (end 138.3401 112.7426) (width 0.6096) (layer "F.Cu") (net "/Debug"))
 (segment (start 149.7701 101.3126) (end 159.9301 101.3126) (width 0.6096) (layer "F.Cu") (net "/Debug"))
 (segment (start 138.3401 112.7426) (end 149.7701 101.3126) (width 0.6096) (layer "F.Cu") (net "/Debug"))
 (via (at 162.8701 101.3126) (size 1.9304) (drill 1) (layers "F.Cu" "B.Cu") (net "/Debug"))
 (segment (start 162.97 101.3) (end 160.03 101.3) (width 0.6096) (layer "B.Cu") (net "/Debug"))
 (segment (start 133.0781 104.9406) (end 135.8001 108.9326) (width 0.6096) (layer "F.Cu") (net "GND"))
 (segment (start 131.6 101.4) (end 131.2 101.4) (width 0.6096) (layer "F.Cu") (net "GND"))
 (segment (start 144.6901 108.9326) (end 154.8501 108.9326) (width 0.6096) (layer "F.Cu") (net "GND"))
 (segment (start 131.2 101.4) (end 130 102.6) (width 0.6096) (layer "F.Cu") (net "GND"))
 (segment (start 140.8801 124.6726) (end 140.8801 112.7426) (width 0.6096) (layer "F.Cu") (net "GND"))
 (segment (start 154.8501 108.9326) (end 159.9301 103.8526) (width 0.6096) (layer "F.Cu") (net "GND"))
 (segment (start 140.8801 112.7426) (end 144.6901 108.9326) (width 0.6096) (layer "F.Cu") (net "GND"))
 (segment (start 135.8001 108.9326) (end 139.6101 108.9326) (width 0.6096) (layer "F.Cu") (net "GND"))
 (segment (start 131.2281 104.9406) (end 133.0781 104.9406) (width 0.6096) (layer "F.Cu") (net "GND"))
 (via (at 130 102.6) (size 1.108) (drill 0.6) (layers "F.Cu" "B.Cu") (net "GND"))
 (via (at 139.6101 108.9326) (size 1.108) (drill 0.6) (layers "F.Cu" "B.Cu") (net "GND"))
 (via (at 144.6901 108.9326) (size 1.108) (drill 0.6) (layers "F.Cu" "B.Cu") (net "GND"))
 (via (at 162.8701 103.8526) (size 1.9304) (drill 1) (layers "F.Cu" "B.Cu") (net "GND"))
 (segment (start 162.87 103.9) (end 159.93 103.9) (width 0.6096) (layer "B.Cu") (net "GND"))
 (segment (start 130 103.7125) (end 131.2281 104.9406) (width 0.6096) (layer "B.Cu") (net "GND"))
 (segment (start 130 102.6) (end 130 103.7125) (width 0.6096) (layer "B.Cu") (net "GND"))
 (segment (start 139.6101 108.9326) (end 144.6901 108.9326) (width 0.6096) (layer "B.Cu") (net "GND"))
 (segment (start 133.6 101.4) (end 133.6 103.7002) (width 0.6096) (layer "F.Cu") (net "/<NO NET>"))
 (segment (start 136.8669 103.7002) (end 133.6 103.7002) (width 0.6096) (layer "F.Cu") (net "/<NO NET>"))
 (segment (start 131.2 106.4) (end 130 106.4) (width 0.6096) (layer "F.Cu") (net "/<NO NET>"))
 (segment (start 130 106.4) (end 129.5 105.9) (width 0.6096) (layer "F.Cu") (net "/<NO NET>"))
 (segment (start 130.9233 106.291) (end 131.2281 106.291) (width 0.6096) (layer "F.Cu") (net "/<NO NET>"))
 (segment (start 131.2281 106.291) (end 131.2281 106.4406) (width 0.6096) (layer "F.Cu") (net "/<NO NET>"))
 (segment (start 137.0193 103.8526) (end 137.0701 103.8526) (width 0.6096) (layer "F.Cu") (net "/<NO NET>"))
 (segment (start 133.6 103.7002) (end 130.7709 103.7002) (width 0.6096) (layer "F.Cu") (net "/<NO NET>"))
 (segment (start 130.2998 103.7002) (end 130.7709 103.7002) (width 0.6096) (layer "F.Cu") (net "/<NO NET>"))
 (segment (start 129.5 105.9) (end 129.5 104.5) (width 0.6096) (layer "F.Cu") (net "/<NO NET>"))
 (segment (start 137.0193 103.8526) (end 136.8669 103.7002) (width 0.6096) (layer "F.Cu") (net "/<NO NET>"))
 (segment (start 129.5 104.5) (end 130.2998 103.7002) (width 0.6096) (layer "F.Cu") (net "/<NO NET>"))
 (segment (start 134.16 88.6) (end 134.1 88.66) (width 0.2) (layer "F.Cu") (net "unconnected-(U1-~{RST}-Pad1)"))
 (via (at 134.1 88.66) (size 1.9304) (drill 1) (layers "F.Cu" "B.Cu") (free yes) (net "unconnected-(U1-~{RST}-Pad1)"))
 (segment (start 137.1 88.6) (end 134.16 88.6) (width 0.6096) (layer "B.Cu") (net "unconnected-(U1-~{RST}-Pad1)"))
 (via (at 134.1 91.2) (size 1.9304) (drill 1) (layers "F.Cu" "B.Cu") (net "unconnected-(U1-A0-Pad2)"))
 (segment (start 137.17 91.2) (end 134.23 91.2) (width 0.6096) (layer "B.Cu") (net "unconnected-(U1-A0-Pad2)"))
 (via (at 134.1 93.74) (size 1.9304) (drill 1) (layers "F.Cu" "B.Cu") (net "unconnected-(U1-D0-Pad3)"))
 (segment (start 137.07 93.7) (end 134.13 93.7) (width 0.6096) (layer "B.Cu") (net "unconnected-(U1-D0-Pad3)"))
 (via (at 134.1 96.28) (size 1.9304) (drill 1) (layers "F.Cu" "B.Cu") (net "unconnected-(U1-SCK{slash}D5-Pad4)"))
 (segment (start 137.07 96.3) (end 134.13 96.3) (width 0.6096) (layer "B.Cu") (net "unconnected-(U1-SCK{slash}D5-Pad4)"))
 (via (at 134.1 98.82) (size 1.9304) (drill 1) (layers "F.Cu" "B.Cu") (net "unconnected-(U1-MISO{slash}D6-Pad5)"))
 (segment (start 137.07 98.8) (end 134.13 98.8) (width 0.6096) (layer "B.Cu") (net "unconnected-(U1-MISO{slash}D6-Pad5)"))
 (segment (start 131.2281 107.9406) (end 132.9821 107.9406) (width 0.6096) (layer "B.Cu") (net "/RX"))
 (segment (start 132.9821 107.9406) (end 134.5301 106.3926) (width 0.6096) (layer "B.Cu") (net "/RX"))
 (segment (start 134.5301 103.8526) (end 137.0701 101.3126) (width 0.6096) (layer "B.Cu") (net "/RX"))
 (segment (start 134.5301 106.3926) (end 134.5301 103.8526) (width 0.6096) (layer "B.Cu") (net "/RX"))
 (via (at 162.8701 106.3926) (size 1.9304) (drill 1) (layers "F.Cu" "B.Cu") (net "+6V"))
 (segment (start 133.2601 110.2026) (end 156.1201 110.2026) (width 0.6096) (layer "B.Cu") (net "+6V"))
 (segment (start 162.87 106.4) (end 159.93 106.4) (width 0.6096) (layer "B.Cu") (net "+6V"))
 (segment (start 131.2281 109.4406) (end 132.4981 109.4406) (width 0.6096) (layer "B.Cu") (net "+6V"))
 (segment (start 156.1201 110.2026) (end 159.9301 106.3926) (width 0.6096) (layer "B.Cu") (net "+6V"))
 (segment (start 132.4981 109.4406) (end 133.2601 110.2026) (width 0.6096) (layer "B.Cu") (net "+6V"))
 (via (at 162.8701 98.7726) (size 1.9304) (drill 1) (layers "F.Cu" "B.Cu") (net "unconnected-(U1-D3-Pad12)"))
 (segment (start 162.97 98.8) (end 160.03 98.8) (width 0.6096) (layer "B.Cu") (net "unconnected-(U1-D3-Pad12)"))
 (via (at 162.8701 96.2326) (size 1.9304) (drill 1) (layers "F.Cu" "B.Cu") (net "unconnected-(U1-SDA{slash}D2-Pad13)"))
 (segment (start 162.87 96.2) (end 159.93 96.2) (width 0.6096) (layer "B.Cu") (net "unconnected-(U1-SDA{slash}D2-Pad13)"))
 (via (at 162.8701 93.6926) (size 1.9304) (drill 1) (layers "F.Cu" "B.Cu") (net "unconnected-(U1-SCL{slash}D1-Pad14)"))
 (segment (start 162.97 93.7) (end 160.03 93.7) (width 0.6096) (layer "B.Cu") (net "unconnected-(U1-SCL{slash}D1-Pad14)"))
 (via (at 162.8701 91.1526) (size 1.9304) (drill 1) (layers "F.Cu" "B.Cu") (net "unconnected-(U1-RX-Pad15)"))
 (segment (start 162.87 91.1) (end 159.93 91.1) (width 0.6096) (layer "B.Cu") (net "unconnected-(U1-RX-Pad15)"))
 (via (at 162.8701 88.6126) (size 1.9304) (drill 1) (layers "F.Cu" "B.Cu") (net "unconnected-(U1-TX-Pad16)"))
 (segment (start 162.87 88.6) (end 159.93 88.6) (width 0.6096) (layer "B.Cu") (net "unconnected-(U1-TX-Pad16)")))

